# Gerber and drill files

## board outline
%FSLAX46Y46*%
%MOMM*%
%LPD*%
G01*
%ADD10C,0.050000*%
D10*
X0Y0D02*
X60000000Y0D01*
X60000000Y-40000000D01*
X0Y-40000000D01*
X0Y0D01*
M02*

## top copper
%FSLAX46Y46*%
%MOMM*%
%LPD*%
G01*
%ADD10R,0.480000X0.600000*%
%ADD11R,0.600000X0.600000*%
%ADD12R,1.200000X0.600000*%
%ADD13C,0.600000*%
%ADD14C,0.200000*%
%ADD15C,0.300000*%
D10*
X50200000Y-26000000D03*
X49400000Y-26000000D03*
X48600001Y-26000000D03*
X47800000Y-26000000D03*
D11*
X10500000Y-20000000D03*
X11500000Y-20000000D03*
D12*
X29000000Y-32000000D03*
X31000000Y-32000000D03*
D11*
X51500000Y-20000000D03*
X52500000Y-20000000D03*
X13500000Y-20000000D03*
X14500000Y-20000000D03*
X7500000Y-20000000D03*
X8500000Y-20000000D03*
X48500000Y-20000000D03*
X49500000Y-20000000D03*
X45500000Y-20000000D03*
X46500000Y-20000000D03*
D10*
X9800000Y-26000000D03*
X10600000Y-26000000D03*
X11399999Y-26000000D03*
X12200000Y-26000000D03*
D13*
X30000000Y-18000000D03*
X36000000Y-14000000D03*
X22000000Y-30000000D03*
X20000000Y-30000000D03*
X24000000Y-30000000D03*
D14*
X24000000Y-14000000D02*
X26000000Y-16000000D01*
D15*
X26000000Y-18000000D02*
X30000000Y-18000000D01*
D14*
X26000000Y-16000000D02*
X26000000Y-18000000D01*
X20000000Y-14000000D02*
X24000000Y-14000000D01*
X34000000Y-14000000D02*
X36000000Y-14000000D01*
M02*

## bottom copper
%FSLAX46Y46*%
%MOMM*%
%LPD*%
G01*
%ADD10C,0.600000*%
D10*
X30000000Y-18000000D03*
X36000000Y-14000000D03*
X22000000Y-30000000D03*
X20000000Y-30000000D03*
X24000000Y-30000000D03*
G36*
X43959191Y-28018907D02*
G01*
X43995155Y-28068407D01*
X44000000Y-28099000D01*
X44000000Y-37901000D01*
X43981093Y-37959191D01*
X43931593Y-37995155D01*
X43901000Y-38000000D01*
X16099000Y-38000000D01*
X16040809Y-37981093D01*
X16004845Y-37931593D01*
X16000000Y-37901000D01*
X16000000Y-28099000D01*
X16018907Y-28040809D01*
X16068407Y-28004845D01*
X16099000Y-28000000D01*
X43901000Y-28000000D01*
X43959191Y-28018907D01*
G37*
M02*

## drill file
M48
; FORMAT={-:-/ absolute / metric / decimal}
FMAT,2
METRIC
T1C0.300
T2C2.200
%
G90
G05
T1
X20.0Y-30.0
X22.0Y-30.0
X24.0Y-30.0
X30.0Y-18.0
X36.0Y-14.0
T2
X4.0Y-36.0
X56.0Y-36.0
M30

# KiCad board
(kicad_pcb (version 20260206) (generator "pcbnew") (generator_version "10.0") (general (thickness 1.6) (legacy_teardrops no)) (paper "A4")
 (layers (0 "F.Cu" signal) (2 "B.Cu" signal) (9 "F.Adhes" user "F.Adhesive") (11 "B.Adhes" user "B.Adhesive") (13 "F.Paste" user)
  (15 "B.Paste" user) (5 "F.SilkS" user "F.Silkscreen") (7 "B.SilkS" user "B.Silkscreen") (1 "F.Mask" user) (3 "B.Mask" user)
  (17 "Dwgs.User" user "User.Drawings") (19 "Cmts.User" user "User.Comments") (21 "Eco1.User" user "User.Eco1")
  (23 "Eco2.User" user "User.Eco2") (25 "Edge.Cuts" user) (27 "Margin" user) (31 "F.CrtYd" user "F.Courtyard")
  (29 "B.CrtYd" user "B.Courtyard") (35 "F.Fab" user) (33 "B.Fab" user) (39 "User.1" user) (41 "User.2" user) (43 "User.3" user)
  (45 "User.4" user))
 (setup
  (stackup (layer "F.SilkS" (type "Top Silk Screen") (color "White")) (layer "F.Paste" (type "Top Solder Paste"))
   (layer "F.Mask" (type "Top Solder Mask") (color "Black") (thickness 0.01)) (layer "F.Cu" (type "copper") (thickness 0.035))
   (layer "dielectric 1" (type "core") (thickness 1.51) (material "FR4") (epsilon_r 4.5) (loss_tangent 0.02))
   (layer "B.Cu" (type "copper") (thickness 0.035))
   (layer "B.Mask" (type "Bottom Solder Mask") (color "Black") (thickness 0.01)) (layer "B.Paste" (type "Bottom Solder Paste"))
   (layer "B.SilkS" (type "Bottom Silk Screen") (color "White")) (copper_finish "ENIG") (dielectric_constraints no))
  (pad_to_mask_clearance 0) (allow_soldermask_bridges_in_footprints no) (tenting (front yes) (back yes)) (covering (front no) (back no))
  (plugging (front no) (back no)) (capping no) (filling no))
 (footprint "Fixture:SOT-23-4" (layer "F.Cu") (at 49 26 180)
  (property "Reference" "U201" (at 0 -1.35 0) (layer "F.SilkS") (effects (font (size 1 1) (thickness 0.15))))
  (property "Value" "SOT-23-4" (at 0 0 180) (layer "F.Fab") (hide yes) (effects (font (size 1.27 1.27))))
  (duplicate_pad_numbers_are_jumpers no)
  (pad "1" smd rect (at -1.2 0 180) (size 0.48 0.6) (layers "F.Cu" "F.Mask" "F.Paste") (thermal_bridge_angle 45))
  (pad "2" smd rect (at -0.4 0 180) (size 0.48 0.6) (layers "F.Cu" "F.Mask" "F.Paste") (thermal_bridge_angle 45))
  (pad "3" smd rect (at 0.399999 0 180) (size 0.48 0.6) (layers "F.Cu" "F.Mask" "F.Paste") (thermal_bridge_angle 45))
  (pad "4" smd rect (at 1.2 0 180) (size 0.48 0.6) (layers "F.Cu" "F.Mask" "F.Paste") (thermal_bridge_angle 45)))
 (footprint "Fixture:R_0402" (layer "F.Cu") (at 11 20)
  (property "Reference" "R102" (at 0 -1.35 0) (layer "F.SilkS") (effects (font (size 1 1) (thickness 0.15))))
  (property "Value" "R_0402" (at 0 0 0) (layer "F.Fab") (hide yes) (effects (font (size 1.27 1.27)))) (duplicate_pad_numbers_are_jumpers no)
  (pad "1" smd rect (at -0.5 0) (size 0.6 0.6) (layers "F.Cu" "F.Mask" "F.Paste") (thermal_bridge_angle 45))
  (pad "2" smd rect (at 0.5 0) (size 0.6 0.6) (layers "F.Cu" "F.Mask" "F.Paste") (thermal_bridge_angle 45)))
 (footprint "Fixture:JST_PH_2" (layer "F.Cu") (at 30 32)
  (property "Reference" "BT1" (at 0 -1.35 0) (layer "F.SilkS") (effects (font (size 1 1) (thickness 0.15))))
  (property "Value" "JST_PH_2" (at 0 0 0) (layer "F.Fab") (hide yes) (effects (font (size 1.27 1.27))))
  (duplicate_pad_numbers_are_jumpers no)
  (pad "1" smd rect (at -1 0) (size 1.2 0.6) (layers "F.Cu" "F.Mask" "F.Paste") (thermal_bridge_angle 45))
  (pad "2" smd rect (at 1 0) (size 1.2 0.6) (layers "F.Cu" "F.Mask" "F.Paste") (thermal_bridge_angle 45)))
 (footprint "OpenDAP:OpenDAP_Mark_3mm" (layer "F.Cu") (at 52 3)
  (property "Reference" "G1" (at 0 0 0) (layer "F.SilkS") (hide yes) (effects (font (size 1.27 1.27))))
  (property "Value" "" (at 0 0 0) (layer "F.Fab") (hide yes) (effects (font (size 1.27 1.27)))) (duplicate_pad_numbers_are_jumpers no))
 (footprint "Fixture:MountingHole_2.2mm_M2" (layer "F.Cu") (at 56 36)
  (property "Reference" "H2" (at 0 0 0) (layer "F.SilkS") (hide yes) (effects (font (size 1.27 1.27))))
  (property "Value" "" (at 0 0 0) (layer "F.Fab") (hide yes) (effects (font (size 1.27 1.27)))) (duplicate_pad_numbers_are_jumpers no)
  (pad "" np_thru_hole circle (at 0 0) (size 2.2 2.2) (drill 2.2) (layers "*.Cu" "*.Mask")))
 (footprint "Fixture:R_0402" (layer "F.Cu") (at 52 20)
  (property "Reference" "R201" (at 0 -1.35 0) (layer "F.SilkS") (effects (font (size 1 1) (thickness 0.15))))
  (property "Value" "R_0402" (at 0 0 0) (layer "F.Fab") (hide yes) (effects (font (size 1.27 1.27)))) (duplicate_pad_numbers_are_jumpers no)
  (pad "1" smd rect (at -0.5 0) (size 0.6 0.6) (layers "F.Cu" "F.Mask" "F.Paste") (thermal_bridge_angle 45))
  (pad "2" smd rect (at 0.5 0) (size 0.6 0.6) (layers "F.Cu" "F.Mask" "F.Paste") (thermal_bridge_angle 45)))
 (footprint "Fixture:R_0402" (layer "F.Cu") (at 14 20)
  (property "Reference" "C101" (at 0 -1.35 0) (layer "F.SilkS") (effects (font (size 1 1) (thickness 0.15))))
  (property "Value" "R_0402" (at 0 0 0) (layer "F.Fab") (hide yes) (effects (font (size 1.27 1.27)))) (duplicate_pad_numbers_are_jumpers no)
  (pad "1" smd rect (at -0.5 0) (size 0.6 0.6) (layers "F.Cu" "F.Mask" "F.Paste") (thermal_bridge_angle 45))
  (pad "2" smd rect (at 0.5 0) (size 0.6 0.6) (layers "F.Cu" "F.Mask" "F.Paste") (thermal_bridge_angle 45)))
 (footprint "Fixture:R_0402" (layer "F.Cu") (at 8 20)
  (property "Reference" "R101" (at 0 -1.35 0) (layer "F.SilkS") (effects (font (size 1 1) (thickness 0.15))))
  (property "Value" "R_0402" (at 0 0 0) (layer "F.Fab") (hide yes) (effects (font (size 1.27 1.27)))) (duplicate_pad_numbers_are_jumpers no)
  (pad "1" smd rect (at -0.5 0) (size 0.6 0.6) (layers "F.Cu" "F.Mask" "F.Paste") (thermal_bridge_angle 45))
  (pad "2" smd rect (at 0.5 0) (size 0.6 0.6) (layers "F.Cu" "F.Mask" "F.Paste") (thermal_bridge_angle 45)))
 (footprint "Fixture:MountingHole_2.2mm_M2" (layer "F.Cu") (at 4 36)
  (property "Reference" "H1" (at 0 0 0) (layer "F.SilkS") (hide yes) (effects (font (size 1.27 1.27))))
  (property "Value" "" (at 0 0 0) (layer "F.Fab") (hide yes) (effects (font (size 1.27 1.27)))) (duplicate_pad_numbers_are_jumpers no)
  (pad "" np_thru_hole circle (at 0 0) (size 2.2 2.2) (drill 2.2) (layers "*.Cu" "*.Mask")))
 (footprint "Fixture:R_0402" (layer "F.Cu") (at 49 20)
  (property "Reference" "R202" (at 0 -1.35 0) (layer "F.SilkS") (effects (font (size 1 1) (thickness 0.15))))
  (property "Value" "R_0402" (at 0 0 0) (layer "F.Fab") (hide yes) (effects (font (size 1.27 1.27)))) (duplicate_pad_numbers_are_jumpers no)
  (pad "1" smd rect (at -0.5 0) (size 0.6 0.6) (layers "F.Cu" "F.Mask" "F.Paste") (thermal_bridge_angle 45))
  (pad "2" smd rect (at 0.5 0) (size 0.6 0.6) (layers "F.Cu" "F.Mask" "F.Paste") (thermal_bridge_angle 45)))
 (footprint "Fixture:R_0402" (layer "F.Cu") (at 46 20)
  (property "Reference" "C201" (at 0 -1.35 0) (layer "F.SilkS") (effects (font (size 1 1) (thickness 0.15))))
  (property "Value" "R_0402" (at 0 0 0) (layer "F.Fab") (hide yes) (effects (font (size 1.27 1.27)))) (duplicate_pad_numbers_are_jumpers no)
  (pad "1" smd rect (at -0.5 0) (size 0.6 0.6) (layers "F.Cu" "F.Mask" "F.Paste") (thermal_bridge_angle 45))
  (pad "2" smd rect (at 0.5 0) (size 0.6 0.6) (layers "F.Cu" "F.Mask" "F.Paste") (thermal_bridge_angle 45)))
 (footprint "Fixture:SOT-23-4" (layer "F.Cu") (at 11 26)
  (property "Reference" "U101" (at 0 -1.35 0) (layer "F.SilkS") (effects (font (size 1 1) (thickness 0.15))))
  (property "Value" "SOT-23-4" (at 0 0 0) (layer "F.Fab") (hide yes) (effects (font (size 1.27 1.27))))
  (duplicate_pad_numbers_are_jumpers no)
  (pad "1" smd rect (at -1.2 0) (size 0.48 0.6) (layers "F.Cu" "F.Mask" "F.Paste") (thermal_bridge_angle 45))
  (pad "2" smd rect (at -0.4 0) (size 0.48 0.6) (layers "F.Cu" "F.Mask" "F.Paste") (thermal_bridge_angle 45))
  (pad "3" smd rect (at 0.399999 0) (size 0.48 0.6) (layers "F.Cu" "F.Mask" "F.Paste") (thermal_bridge_angle 45))
  (pad "4" smd rect (at 1.2 0) (size 0.48 0.6) (layers "F.Cu" "F.Mask" "F.Paste") (thermal_bridge_angle 45)))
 (gr_rect (start 0 0) (end 60 40) (stroke (width 0.05) (type default)) (fill no) (layer "Edge.Cuts"))
 (segment (start 24 14) (end 26 16) (width 0.2) (layer "F.Cu") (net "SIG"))
 (segment (start 26 18) (end 30 18) (width 0.3) (layer "F.Cu") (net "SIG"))
 (segment (start 26 16) (end 26 18) (width 0.2) (layer "F.Cu") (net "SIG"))
 (segment (start 20 14) (end 24 14) (width 0.2) (layer "F.Cu") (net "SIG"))
 (via (at 30 18) (size 0.6) (drill 0.3) (layers "F.Cu" "B.Cu") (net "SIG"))
 (segment (start 34 14) (end 36 14) (width 0.2) (layer "F.Cu") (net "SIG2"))
 (via (at 36 14) (size 0.6) (drill 0.3) (layers "F.Cu" "B.Cu") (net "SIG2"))
 (via (at 22 30) (size 0.6) (drill 0.3) (layers "F.Cu" "B.Cu") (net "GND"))
 (via (at 20 30) (size 0.6) (drill 0.3) (layers "F.Cu" "B.Cu") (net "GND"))
 (via (at 24 30) (size 0.6) (drill 0.3) (layers "F.Cu" "B.Cu") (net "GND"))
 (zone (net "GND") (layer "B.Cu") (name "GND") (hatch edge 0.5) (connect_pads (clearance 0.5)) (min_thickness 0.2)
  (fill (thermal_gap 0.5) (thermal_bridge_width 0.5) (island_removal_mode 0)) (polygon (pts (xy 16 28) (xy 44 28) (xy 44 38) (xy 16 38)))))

